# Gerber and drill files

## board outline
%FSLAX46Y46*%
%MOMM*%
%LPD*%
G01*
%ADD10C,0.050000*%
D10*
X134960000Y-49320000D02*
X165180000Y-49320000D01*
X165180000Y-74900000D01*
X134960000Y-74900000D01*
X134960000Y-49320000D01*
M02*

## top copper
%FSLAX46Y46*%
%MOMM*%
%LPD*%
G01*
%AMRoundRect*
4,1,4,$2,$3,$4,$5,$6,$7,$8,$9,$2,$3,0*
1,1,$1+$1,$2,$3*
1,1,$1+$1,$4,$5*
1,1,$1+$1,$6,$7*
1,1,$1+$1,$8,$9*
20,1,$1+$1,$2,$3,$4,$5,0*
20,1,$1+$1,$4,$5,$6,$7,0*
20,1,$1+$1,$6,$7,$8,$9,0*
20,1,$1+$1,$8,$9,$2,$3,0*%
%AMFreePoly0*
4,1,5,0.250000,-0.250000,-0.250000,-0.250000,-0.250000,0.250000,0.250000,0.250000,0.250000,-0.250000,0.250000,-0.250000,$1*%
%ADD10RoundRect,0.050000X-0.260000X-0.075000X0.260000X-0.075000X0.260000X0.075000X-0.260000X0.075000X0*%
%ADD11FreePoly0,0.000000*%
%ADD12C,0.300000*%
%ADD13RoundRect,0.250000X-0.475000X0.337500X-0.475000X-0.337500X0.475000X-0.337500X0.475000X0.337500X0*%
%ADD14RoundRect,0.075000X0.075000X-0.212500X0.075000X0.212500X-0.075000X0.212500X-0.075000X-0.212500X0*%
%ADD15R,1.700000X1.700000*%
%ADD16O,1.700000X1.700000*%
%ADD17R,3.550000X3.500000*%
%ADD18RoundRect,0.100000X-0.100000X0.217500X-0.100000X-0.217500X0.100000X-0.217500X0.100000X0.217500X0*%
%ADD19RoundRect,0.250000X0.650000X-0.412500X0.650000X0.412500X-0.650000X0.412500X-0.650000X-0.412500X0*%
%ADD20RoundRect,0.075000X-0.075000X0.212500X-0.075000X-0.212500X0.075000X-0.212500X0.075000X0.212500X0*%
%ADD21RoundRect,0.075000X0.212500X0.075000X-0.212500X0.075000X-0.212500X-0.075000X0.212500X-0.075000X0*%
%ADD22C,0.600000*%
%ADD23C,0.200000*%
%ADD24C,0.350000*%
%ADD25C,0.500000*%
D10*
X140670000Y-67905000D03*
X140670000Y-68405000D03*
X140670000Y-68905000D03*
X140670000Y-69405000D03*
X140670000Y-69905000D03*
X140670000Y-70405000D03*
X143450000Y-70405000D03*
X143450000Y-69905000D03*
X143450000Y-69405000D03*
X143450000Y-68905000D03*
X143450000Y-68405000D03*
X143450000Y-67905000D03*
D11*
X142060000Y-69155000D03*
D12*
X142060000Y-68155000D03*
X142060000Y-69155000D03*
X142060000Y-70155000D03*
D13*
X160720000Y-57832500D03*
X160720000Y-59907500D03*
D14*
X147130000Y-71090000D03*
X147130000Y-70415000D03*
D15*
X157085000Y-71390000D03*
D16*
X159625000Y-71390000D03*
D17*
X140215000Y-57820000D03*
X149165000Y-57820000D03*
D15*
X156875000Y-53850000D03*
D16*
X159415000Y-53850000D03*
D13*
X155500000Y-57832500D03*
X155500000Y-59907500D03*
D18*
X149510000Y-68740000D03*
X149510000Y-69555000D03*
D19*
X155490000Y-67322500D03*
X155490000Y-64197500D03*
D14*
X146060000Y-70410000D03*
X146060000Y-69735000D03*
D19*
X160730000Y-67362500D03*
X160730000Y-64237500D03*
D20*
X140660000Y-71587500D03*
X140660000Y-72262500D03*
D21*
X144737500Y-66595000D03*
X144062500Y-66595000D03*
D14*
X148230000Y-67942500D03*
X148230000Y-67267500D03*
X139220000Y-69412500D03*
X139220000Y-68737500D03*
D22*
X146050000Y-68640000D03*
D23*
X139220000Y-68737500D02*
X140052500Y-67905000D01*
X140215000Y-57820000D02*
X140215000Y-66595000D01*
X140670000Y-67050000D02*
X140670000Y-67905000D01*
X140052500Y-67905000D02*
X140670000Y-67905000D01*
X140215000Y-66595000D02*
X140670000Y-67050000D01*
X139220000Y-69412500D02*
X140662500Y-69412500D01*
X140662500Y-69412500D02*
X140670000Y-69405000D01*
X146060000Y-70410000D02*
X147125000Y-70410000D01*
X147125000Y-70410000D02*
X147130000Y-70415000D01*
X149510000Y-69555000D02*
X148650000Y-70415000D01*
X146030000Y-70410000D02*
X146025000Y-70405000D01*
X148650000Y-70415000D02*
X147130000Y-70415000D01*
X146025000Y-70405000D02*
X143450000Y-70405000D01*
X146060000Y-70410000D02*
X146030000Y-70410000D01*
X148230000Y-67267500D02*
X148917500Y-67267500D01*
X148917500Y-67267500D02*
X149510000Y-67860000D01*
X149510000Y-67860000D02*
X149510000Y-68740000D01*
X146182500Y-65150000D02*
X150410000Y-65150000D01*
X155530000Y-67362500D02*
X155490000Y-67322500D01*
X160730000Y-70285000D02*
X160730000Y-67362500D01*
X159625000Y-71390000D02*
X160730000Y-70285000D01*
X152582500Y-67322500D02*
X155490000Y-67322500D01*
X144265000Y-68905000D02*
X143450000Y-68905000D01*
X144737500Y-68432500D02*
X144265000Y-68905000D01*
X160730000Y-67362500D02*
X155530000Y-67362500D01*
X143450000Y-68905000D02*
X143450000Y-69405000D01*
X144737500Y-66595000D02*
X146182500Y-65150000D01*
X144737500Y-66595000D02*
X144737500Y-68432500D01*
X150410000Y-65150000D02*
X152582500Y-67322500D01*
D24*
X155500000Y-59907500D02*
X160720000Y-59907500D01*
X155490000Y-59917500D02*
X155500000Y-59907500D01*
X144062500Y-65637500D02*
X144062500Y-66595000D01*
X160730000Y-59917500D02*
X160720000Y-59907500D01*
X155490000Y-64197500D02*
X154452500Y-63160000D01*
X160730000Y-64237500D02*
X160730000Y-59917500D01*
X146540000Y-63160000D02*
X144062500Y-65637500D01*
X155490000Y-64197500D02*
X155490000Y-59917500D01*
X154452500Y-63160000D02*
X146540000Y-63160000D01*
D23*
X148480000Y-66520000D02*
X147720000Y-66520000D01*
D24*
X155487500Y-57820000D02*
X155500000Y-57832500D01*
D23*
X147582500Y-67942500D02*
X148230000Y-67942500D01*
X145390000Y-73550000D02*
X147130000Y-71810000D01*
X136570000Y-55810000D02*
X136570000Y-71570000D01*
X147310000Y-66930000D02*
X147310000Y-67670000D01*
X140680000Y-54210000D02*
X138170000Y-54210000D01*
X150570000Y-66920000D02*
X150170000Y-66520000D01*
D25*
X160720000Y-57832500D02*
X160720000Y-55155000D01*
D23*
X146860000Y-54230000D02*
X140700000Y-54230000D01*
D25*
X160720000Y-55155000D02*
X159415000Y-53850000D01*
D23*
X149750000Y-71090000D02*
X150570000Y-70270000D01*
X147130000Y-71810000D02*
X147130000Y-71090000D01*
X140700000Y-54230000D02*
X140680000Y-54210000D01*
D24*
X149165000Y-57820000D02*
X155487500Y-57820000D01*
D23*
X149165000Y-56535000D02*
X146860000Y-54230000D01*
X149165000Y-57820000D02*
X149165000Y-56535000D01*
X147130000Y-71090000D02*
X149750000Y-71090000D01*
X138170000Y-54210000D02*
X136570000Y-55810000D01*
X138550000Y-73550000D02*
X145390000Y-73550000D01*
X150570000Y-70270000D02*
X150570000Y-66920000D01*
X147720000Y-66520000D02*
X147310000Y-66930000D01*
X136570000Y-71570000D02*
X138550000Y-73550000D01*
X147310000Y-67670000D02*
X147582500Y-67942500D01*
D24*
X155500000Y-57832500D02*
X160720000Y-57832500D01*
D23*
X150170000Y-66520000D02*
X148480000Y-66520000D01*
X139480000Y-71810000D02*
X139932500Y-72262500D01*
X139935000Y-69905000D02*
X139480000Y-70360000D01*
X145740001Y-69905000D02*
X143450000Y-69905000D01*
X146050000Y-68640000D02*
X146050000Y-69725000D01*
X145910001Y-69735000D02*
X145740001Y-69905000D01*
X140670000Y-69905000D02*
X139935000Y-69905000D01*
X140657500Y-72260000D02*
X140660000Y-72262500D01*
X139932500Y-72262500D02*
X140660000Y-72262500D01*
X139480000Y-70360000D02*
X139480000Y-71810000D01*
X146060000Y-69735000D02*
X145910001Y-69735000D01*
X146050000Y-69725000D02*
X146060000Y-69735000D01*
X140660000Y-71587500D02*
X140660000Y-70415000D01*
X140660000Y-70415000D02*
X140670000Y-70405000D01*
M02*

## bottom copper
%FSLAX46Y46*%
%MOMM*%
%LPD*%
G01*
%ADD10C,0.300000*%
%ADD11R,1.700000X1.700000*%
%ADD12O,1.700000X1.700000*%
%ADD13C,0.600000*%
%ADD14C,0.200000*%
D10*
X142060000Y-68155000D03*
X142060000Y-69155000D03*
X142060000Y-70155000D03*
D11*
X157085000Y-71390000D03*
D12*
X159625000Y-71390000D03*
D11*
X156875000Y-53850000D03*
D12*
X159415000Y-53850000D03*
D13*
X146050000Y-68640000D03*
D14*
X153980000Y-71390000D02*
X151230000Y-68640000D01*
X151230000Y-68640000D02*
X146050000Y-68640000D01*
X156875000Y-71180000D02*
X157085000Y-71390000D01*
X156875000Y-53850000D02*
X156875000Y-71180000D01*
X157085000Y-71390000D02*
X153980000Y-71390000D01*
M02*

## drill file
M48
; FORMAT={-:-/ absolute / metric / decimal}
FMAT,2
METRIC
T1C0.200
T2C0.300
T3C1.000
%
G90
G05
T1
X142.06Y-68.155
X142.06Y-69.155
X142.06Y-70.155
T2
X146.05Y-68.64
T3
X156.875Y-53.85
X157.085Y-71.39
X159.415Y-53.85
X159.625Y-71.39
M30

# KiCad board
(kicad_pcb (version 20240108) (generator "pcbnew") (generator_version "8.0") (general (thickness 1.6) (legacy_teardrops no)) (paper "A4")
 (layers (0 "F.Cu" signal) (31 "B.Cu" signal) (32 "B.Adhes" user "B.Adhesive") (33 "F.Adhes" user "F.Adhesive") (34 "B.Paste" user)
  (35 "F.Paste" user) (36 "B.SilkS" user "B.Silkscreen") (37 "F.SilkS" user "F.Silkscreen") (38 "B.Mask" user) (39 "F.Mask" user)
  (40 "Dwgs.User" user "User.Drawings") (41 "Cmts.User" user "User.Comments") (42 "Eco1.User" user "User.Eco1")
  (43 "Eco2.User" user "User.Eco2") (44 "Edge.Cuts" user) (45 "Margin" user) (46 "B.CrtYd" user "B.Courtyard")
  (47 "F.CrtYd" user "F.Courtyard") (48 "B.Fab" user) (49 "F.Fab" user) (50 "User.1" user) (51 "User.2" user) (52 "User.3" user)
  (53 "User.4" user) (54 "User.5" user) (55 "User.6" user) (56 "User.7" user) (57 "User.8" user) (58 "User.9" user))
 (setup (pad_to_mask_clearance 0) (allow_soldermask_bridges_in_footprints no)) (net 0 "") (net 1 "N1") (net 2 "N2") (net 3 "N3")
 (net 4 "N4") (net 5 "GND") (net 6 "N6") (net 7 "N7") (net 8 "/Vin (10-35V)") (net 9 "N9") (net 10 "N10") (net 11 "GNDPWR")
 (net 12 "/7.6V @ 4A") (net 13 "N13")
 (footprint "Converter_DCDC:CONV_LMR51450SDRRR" (layer "F.Cu") (at 142.06 69.155)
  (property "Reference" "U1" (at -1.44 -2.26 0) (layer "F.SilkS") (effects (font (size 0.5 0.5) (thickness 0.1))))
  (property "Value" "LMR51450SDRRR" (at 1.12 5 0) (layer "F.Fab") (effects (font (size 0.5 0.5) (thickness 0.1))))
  (pad "1" smd roundrect (at -1.39 -1.25) (size 0.62 0.25) (layers "F.Cu" "F.Paste") (roundrect_rratio 0.2) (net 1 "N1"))
  (pad "2" smd roundrect (at -1.39 -0.75) (size 0.62 0.25) (layers "F.Cu" "F.Paste") (roundrect_rratio 0.2) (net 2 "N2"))
  (pad "3" smd roundrect (at -1.39 -0.25) (size 0.62 0.25) (layers "F.Cu" "F.Paste") (roundrect_rratio 0.2) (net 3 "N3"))
  (pad "4" smd roundrect (at -1.39 0.25) (size 0.62 0.25) (layers "F.Cu" "F.Paste") (roundrect_rratio 0.2) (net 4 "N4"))
  (pad "5" smd roundrect (at -1.39 0.75) (size 0.62 0.25) (layers "F.Cu" "F.Paste") (roundrect_rratio 0.2) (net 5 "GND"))
  (pad "6" smd roundrect (at -1.39 1.25) (size 0.62 0.25) (layers "F.Cu" "F.Paste") (roundrect_rratio 0.2) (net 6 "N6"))
  (pad "7" smd roundrect (at 1.39 1.25) (size 0.62 0.25) (layers "F.Cu" "F.Paste") (roundrect_rratio 0.2) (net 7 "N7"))
  (pad "8" smd roundrect (at 1.39 0.75) (size 0.62 0.25) (layers "F.Cu" "F.Paste") (roundrect_rratio 0.2) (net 5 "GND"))
  (pad "9" smd roundrect (at 1.39 0.25) (size 0.62 0.25) (layers "F.Cu" "F.Paste") (roundrect_rratio 0.2) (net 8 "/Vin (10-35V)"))
  (pad "10" smd roundrect (at 1.39 -0.25) (size 0.62 0.25) (layers "F.Cu" "F.Paste") (roundrect_rratio 0.2) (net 8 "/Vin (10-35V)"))
  (pad "11" smd roundrect (at 1.39 -0.75) (size 0.62 0.25) (layers "F.Cu" "F.Paste") (roundrect_rratio 0.2) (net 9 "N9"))
  (pad "12" smd roundrect (at 1.39 -1.25) (size 0.62 0.25) (layers "F.Cu" "F.Paste") (roundrect_rratio 0.2) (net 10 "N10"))
  (pad "13" smd custom (at 0 0) (size 0.5 0.5) (layers "F.Cu") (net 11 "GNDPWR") (options (clearance outline) (anchor rect)) (primitives))
  (pad "14" thru_hole circle (at 0 -1) (size 0.3 0.3) (drill 0.2) (layers "*.Cu") (remove_unused_layers no))
  (pad "15" thru_hole circle (at 0 0) (size 0.3 0.3) (drill 0.2) (layers "*.Cu") (remove_unused_layers no))
  (pad "16" thru_hole circle (at 0 1) (size 0.3 0.3) (drill 0.2) (layers "*.Cu") (remove_unused_layers no)))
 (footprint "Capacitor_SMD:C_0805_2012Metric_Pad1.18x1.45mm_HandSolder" (layer "F.Cu") (at 160.72 58.87 -90)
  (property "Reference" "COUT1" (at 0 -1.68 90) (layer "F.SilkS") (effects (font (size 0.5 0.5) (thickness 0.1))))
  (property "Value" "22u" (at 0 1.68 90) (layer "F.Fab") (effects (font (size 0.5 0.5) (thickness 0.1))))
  (pad "1" smd roundrect (at -1.0375 0 270) (size 1.175 1.45) (layers "F.Cu" "F.Paste" "F.Mask") (roundrect_rratio 0.212766)
   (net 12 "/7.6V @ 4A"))
  (pad "2" smd roundrect (at 1.0375 0 270) (size 1.175 1.45) (layers "F.Cu" "F.Paste" "F.Mask") (roundrect_rratio 0.212766)
   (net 11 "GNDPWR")))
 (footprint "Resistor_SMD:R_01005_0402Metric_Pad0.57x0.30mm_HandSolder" (layer "F.Cu") (at 147.13 70.7525 90)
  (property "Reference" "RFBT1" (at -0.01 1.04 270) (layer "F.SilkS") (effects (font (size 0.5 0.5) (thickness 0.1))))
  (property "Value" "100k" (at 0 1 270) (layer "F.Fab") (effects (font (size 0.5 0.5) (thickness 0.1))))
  (pad "" smd roundrect (at -0.3625 0 90) (size 0.41 0.27) (layers "F.Paste") (roundrect_rratio 0.25))
  (pad "" smd roundrect (at 0.3625 0 90) (size 0.41 0.27) (layers "F.Paste") (roundrect_rratio 0.25))
  (pad "1" smd roundrect (at -0.3375 0 90) (size 0.575 0.3) (layers "F.Cu" "F.Mask") (roundrect_rratio 0.25) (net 12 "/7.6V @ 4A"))
  (pad "2" smd roundrect (at 0.3375 0 90) (size 0.575 0.3) (layers "F.Cu" "F.Mask") (roundrect_rratio 0.25) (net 7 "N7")))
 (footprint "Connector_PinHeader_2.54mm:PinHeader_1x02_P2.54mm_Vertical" (layer "F.Cu") (at 157.085 71.39 90)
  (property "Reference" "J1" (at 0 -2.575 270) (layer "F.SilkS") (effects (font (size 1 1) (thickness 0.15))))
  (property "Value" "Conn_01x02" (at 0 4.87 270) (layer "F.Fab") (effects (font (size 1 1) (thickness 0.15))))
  (pad "1" thru_hole rect (at 0 0 90) (size 1.7 1.7) (drill 1) (layers "*.Cu" "*.Mask") (remove_unused_layers no) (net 5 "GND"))
  (pad "2" thru_hole oval (at 0 2.54 90) (size 1.7 1.7) (drill 1) (layers "*.Cu" "*.Mask") (remove_unused_layers no) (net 8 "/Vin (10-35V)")))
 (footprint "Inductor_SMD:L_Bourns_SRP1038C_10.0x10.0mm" (layer "F.Cu") (at 144.69 57.82)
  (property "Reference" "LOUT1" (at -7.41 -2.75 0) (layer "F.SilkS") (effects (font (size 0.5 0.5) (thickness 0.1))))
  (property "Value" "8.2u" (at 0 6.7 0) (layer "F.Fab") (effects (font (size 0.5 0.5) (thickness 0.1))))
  (pad "1" smd rect (at -4.475 0) (size 3.55 3.5) (layers "F.Cu" "F.Paste" "F.Mask") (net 1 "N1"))
  (pad "2" smd rect (at 4.475 0) (size 3.55 3.5) (layers "F.Cu" "F.Paste" "F.Mask") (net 12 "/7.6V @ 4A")))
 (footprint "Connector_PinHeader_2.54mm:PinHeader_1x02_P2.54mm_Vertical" (layer "F.Cu") (at 156.875 53.85 90)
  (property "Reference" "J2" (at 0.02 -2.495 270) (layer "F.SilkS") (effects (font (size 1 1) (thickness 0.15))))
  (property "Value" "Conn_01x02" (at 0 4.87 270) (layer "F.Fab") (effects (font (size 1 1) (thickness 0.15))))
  (pad "1" thru_hole rect (at 0 0 90) (size 1.7 1.7) (drill 1) (layers "*.Cu" "*.Mask") (remove_unused_layers no) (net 5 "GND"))
  (pad "2" thru_hole oval (at 0 2.54 90) (size 1.7 1.7) (drill 1) (layers "*.Cu" "*.Mask") (remove_unused_layers no) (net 12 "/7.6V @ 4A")))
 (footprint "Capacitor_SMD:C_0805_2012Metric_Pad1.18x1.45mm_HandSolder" (layer "F.Cu") (at 155.5 58.87 -90)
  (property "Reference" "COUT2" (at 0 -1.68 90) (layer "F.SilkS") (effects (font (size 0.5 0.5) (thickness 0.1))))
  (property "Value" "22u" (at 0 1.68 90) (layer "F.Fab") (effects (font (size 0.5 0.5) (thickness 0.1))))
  (pad "1" smd roundrect (at -1.0375 0 270) (size 1.175 1.45) (layers "F.Cu" "F.Paste" "F.Mask") (roundrect_rratio 0.212766)
   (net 12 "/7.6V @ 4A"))
  (pad "2" smd roundrect (at 1.0375 0 270) (size 1.175 1.45) (layers "F.Cu" "F.Paste" "F.Mask") (roundrect_rratio 0.212766)
   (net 11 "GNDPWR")))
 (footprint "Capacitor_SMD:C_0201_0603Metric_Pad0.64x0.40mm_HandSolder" (layer "F.Cu") (at 149.51 69.1475 -90)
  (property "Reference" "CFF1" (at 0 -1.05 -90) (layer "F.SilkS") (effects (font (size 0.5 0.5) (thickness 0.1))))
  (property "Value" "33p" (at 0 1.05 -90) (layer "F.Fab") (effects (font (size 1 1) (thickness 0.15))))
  (pad "" smd roundrect (at -0.4325 0 270) (size 0.458 0.36) (layers "F.Paste") (roundrect_rratio 0.25))
  (pad "" smd roundrect (at 0.4325 0 270) (size 0.458 0.36) (layers "F.Paste") (roundrect_rratio 0.25))
  (pad "1" smd roundrect (at -0.4075 0 270) (size 0.635 0.4) (layers "F.Cu" "F.Mask") (roundrect_rratio 0.25) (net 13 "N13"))
  (pad "2" smd roundrect (at 0.4075 0 270) (size 0.635 0.4) (layers "F.Cu" "F.Mask") (roundrect_rratio 0.25) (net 7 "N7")))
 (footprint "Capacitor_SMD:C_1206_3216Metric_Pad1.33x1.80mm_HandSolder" (layer "F.Cu") (at 155.49 65.76 90)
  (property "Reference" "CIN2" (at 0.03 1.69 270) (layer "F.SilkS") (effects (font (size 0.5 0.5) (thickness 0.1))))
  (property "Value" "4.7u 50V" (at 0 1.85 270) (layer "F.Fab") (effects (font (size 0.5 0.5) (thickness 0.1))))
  (pad "1" smd roundrect (at -1.5625 0 90) (size 1.325 1.8) (layers "F.Cu" "F.Paste" "F.Mask") (roundrect_rratio 0.188679)
   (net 8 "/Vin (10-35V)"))
  (pad "2" smd roundrect (at 1.5625 0 90) (size 1.325 1.8) (layers "F.Cu" "F.Paste" "F.Mask") (roundrect_rratio 0.188679) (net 11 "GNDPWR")))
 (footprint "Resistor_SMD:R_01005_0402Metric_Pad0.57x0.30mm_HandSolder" (layer "F.Cu") (at 146.06 70.0725 90)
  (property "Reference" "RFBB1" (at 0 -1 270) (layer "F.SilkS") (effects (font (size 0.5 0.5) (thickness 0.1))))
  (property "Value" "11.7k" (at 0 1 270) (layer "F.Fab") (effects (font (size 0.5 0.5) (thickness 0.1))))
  (pad "" smd roundrect (at -0.3625 0 90) (size 0.41 0.27) (layers "F.Paste") (roundrect_rratio 0.25))
  (pad "" smd roundrect (at 0.3625 0 90) (size 0.41 0.27) (layers "F.Paste") (roundrect_rratio 0.25))
  (pad "1" smd roundrect (at -0.3375 0 90) (size 0.575 0.3) (layers "F.Cu" "F.Mask") (roundrect_rratio 0.25) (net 7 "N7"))
  (pad "2" smd roundrect (at 0.3375 0 90) (size 0.575 0.3) (layers "F.Cu" "F.Mask") (roundrect_rratio 0.25) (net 5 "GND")))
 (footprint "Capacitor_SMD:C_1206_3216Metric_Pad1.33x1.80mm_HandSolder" (layer "F.Cu") (at 160.73 65.8 90)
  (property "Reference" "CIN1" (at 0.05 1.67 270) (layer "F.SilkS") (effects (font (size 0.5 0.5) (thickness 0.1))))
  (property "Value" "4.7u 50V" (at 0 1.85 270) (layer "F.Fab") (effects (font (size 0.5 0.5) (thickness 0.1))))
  (pad "1" smd roundrect (at -1.5625 0 90) (size 1.325 1.8) (layers "F.Cu" "F.Paste" "F.Mask") (roundrect_rratio 0.188679)
   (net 8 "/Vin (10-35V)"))
  (pad "2" smd roundrect (at 1.5625 0 90) (size 1.325 1.8) (layers "F.Cu" "F.Paste" "F.Mask") (roundrect_rratio 0.188679) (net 11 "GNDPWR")))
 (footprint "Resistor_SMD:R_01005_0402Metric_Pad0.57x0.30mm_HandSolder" (layer "F.Cu") (at 140.66 71.925 -90)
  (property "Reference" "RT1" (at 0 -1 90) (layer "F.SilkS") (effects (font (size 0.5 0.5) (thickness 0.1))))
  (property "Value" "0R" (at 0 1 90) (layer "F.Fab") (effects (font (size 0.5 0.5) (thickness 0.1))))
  (pad "" smd roundrect (at -0.3625 0 270) (size 0.41 0.27) (layers "F.Paste") (roundrect_rratio 0.25))
  (pad "" smd roundrect (at 0.3625 0 270) (size 0.41 0.27) (layers "F.Paste") (roundrect_rratio 0.25))
  (pad "1" smd roundrect (at -0.3375 0 270) (size 0.575 0.3) (layers "F.Cu" "F.Mask") (roundrect_rratio 0.25) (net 6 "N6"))
  (pad "2" smd roundrect (at 0.3375 0 270) (size 0.575 0.3) (layers "F.Cu" "F.Mask") (roundrect_rratio 0.25) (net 5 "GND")))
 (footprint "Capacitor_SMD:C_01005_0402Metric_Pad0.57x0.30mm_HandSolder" (layer "F.Cu") (at 144.4 66.595 180)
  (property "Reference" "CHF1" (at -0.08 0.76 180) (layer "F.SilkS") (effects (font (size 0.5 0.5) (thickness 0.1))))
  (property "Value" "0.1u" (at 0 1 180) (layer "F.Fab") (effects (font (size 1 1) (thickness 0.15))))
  (pad "" smd roundrect (at -0.3625 0 180) (size 0.41 0.27) (layers "F.Paste") (roundrect_rratio 0.25))
  (pad "" smd roundrect (at 0.3625 0 180) (size 0.41 0.27) (layers "F.Paste") (roundrect_rratio 0.25))
  (pad "1" smd roundrect (at -0.3375 0 180) (size 0.575 0.3) (layers "F.Cu" "F.Mask") (roundrect_rratio 0.25) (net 8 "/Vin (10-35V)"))
  (pad "2" smd roundrect (at 0.3375 0 180) (size 0.575 0.3) (layers "F.Cu" "F.Mask") (roundrect_rratio 0.25) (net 11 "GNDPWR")))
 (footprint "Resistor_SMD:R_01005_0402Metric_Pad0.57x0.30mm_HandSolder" (layer "F.Cu") (at 148.23 67.605 90)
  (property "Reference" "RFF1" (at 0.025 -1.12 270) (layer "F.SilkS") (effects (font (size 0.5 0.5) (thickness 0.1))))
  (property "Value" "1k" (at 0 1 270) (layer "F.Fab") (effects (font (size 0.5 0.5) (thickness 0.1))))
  (pad "" smd roundrect (at -0.3625 0 90) (size 0.41 0.27) (layers "F.Paste") (roundrect_rratio 0.25))
  (pad "" smd roundrect (at 0.3625 0 90) (size 0.41 0.27) (layers "F.Paste") (roundrect_rratio 0.25))
  (pad "1" smd roundrect (at -0.3375 0 90) (size 0.575 0.3) (layers "F.Cu" "F.Mask") (roundrect_rratio 0.25) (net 12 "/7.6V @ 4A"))
  (pad "2" smd roundrect (at 0.3375 0 90) (size 0.575 0.3) (layers "F.Cu" "F.Mask") (roundrect_rratio 0.25) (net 13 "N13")))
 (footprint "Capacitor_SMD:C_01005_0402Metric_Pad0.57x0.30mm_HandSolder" (layer "F.Cu") (at 139.22 69.075 90)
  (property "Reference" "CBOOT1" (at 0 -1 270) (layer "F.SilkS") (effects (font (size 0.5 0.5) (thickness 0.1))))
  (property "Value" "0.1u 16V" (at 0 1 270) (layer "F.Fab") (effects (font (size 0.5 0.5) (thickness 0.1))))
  (pad "" smd roundrect (at -0.3625 0 90) (size 0.41 0.27) (layers "F.Paste") (roundrect_rratio 0.25))
  (pad "" smd roundrect (at 0.3625 0 90) (size 0.41 0.27) (layers "F.Paste") (roundrect_rratio 0.25))
  (pad "1" smd roundrect (at -0.3375 0 90) (size 0.575 0.3) (layers "F.Cu" "F.Mask") (roundrect_rratio 0.25) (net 4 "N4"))
  (pad "2" smd roundrect (at 0.3375 0 90) (size 0.575 0.3) (layers "F.Cu" "F.Mask") (roundrect_rratio 0.25) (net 1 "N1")))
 (gr_rect (start 134.96 49.32) (end 165.18 74.9) (stroke (width 0.05) (type default)) (fill none) (layer "Edge.Cuts"))
 (segment (start 139.22 68.7375) (end 140.0525 67.905) (width 0.2) (layer "F.Cu") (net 1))
 (segment (start 140.215 57.82) (end 140.215 66.595) (width 0.2) (layer "F.Cu") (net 1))
 (segment (start 140.67 67.05) (end 140.67 67.905) (width 0.2) (layer "F.Cu") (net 1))
 (segment (start 140.0525 67.905) (end 140.67 67.905) (width 0.2) (layer "F.Cu") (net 1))
 (segment (start 140.215 66.595) (end 140.67 67.05) (width 0.2) (layer "F.Cu") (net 1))
 (segment (start 139.22 69.4125) (end 140.6625 69.4125) (width 0.2) (layer "F.Cu") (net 4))
 (segment (start 140.6625 69.4125) (end 140.67 69.405) (width 0.2) (layer "F.Cu") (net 4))
 (segment (start 146.06 70.41) (end 147.125 70.41) (width 0.2) (layer "F.Cu") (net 7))
 (segment (start 147.125 70.41) (end 147.13 70.415) (width 0.2) (layer "F.Cu") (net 7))
 (segment (start 149.51 69.555) (end 148.65 70.415) (width 0.2) (layer "F.Cu") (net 7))
 (segment (start 146.03 70.41) (end 146.025 70.405) (width 0.2) (layer "F.Cu") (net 7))
 (segment (start 148.65 70.415) (end 147.13 70.415) (width 0.2) (layer "F.Cu") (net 7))
 (segment (start 146.025 70.405) (end 143.45 70.405) (width 0.2) (layer "F.Cu") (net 7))
 (segment (start 146.06 70.41) (end 146.03 70.41) (width 0.2) (layer "F.Cu") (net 7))
 (segment (start 148.23 67.2675) (end 148.9175 67.2675) (width 0.2) (layer "F.Cu") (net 13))
 (segment (start 148.9175 67.2675) (end 149.51 67.86) (width 0.2) (layer "F.Cu") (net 13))
 (segment (start 149.51 67.86) (end 149.51 68.74) (width 0.2) (layer "F.Cu") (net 13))
 (segment (start 146.1825 65.15) (end 150.41 65.15) (width 0.2) (layer "F.Cu") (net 8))
 (segment (start 155.53 67.3625) (end 155.49 67.3225) (width 0.2) (layer "F.Cu") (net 8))
 (segment (start 160.73 70.285) (end 160.73 67.3625) (width 0.2) (layer "F.Cu") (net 8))
 (segment (start 159.625 71.39) (end 160.73 70.285) (width 0.2) (layer "F.Cu") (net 8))
 (segment (start 152.5825 67.3225) (end 155.49 67.3225) (width 0.2) (layer "F.Cu") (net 8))
 (segment (start 144.265 68.905) (end 143.45 68.905) (width 0.2) (layer "F.Cu") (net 8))
 (segment (start 144.7375 68.4325) (end 144.265 68.905) (width 0.2) (layer "F.Cu") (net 8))
 (segment (start 160.73 67.3625) (end 155.53 67.3625) (width 0.2) (layer "F.Cu") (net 8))
 (segment (start 143.45 68.905) (end 143.45 69.405) (width 0.2) (layer "F.Cu") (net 8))
 (segment (start 144.7375 66.595) (end 146.1825 65.15) (width 0.2) (layer "F.Cu") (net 8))
 (segment (start 144.7375 66.595) (end 144.7375 68.4325) (width 0.2) (layer "F.Cu") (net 8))
 (segment (start 150.41 65.15) (end 152.5825 67.3225) (width 0.2) (layer "F.Cu") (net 8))
 (segment (start 155.5 59.9075) (end 160.72 59.9075) (width 0.35) (layer "F.Cu") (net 11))
 (segment (start 155.49 59.9175) (end 155.5 59.9075) (width 0.35) (layer "F.Cu") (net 11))
 (segment (start 144.0625 65.6375) (end 144.0625 66.595) (width 0.35) (layer "F.Cu") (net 11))
 (segment (start 160.73 59.9175) (end 160.72 59.9075) (width 0.35) (layer "F.Cu") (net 11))
 (segment (start 155.49 64.1975) (end 154.4525 63.16) (width 0.35) (layer "F.Cu") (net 11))
 (segment (start 160.73 64.2375) (end 160.73 59.9175) (width 0.35) (layer "F.Cu") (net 11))
 (segment (start 146.54 63.16) (end 144.0625 65.6375) (width 0.35) (layer "F.Cu") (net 11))
 (segment (start 155.49 64.1975) (end 155.49 59.9175) (width 0.35) (layer "F.Cu") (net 11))
 (segment (start 154.4525 63.16) (end 146.54 63.16) (width 0.35) (layer "F.Cu") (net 11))
 (segment (start 148.48 66.52) (end 147.72 66.52) (width 0.2) (layer "F.Cu") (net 12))
 (segment (start 155.4875 57.82) (end 155.5 57.8325) (width 0.35) (layer "F.Cu") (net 12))
 (segment (start 147.5825 67.9425) (end 148.23 67.9425) (width 0.2) (layer "F.Cu") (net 12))
 (segment (start 145.39 73.55) (end 147.13 71.81) (width 0.2) (layer "F.Cu") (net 12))
 (segment (start 136.57 55.81) (end 136.57 71.57) (width 0.2) (layer "F.Cu") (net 12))
 (segment (start 147.31 66.93) (end 147.31 67.67) (width 0.2) (layer "F.Cu") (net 12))
 (segment (start 140.68 54.21) (end 138.17 54.21) (width 0.2) (layer "F.Cu") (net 12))
 (segment (start 150.57 66.92) (end 150.17 66.52) (width 0.2) (layer "F.Cu") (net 12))
 (segment (start 160.72 57.8325) (end 160.72 55.155) (width 0.5) (layer "F.Cu") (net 12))
 (segment (start 146.86 54.23) (end 140.7 54.23) (width 0.2) (layer "F.Cu") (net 12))
 (segment (start 160.72 55.155) (end 159.415 53.85) (width 0.5) (layer "F.Cu") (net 12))
 (segment (start 149.75 71.09) (end 150.57 70.27) (width 0.2) (layer "F.Cu") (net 12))
 (segment (start 147.13 71.81) (end 147.13 71.09) (width 0.2) (layer "F.Cu") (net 12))
 (segment (start 140.7 54.23) (end 140.68 54.21) (width 0.2) (layer "F.Cu") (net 12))
 (segment (start 149.165 57.82) (end 155.4875 57.82) (width 0.35) (layer "F.Cu") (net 12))
 (segment (start 149.165 56.535) (end 146.86 54.23) (width 0.2) (layer "F.Cu") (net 12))
 (segment (start 149.165 57.82) (end 149.165 56.535) (width 0.2) (layer "F.Cu") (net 12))
 (segment (start 147.13 71.09) (end 149.75 71.09) (width 0.2) (layer "F.Cu") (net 12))
 (segment (start 138.17 54.21) (end 136.57 55.81) (width 0.2) (layer "F.Cu") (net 12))
 (segment (start 138.55 73.55) (end 145.39 73.55) (width 0.2) (layer "F.Cu") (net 12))
 (segment (start 150.57 70.27) (end 150.57 66.92) (width 0.2) (layer "F.Cu") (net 12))
 (segment (start 147.72 66.52) (end 147.31 66.93) (width 0.2) (layer "F.Cu") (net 12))
 (segment (start 136.57 71.57) (end 138.55 73.55) (width 0.2) (layer "F.Cu") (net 12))
 (segment (start 147.31 67.67) (end 147.5825 67.9425) (width 0.2) (layer "F.Cu") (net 12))
 (segment (start 155.5 57.8325) (end 160.72 57.8325) (width 0.35) (layer "F.Cu") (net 12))
 (segment (start 150.17 66.52) (end 148.48 66.52) (width 0.2) (layer "F.Cu") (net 12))
 (segment (start 139.48 71.81) (end 139.9325 72.2625) (width 0.2) (layer "F.Cu") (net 5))
 (segment (start 139.935 69.905) (end 139.48 70.36) (width 0.2) (layer "F.Cu") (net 5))
 (segment (start 145.740001 69.905) (end 143.45 69.905) (width 0.2) (layer "F.Cu") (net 5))
 (segment (start 146.05 68.64) (end 146.05 69.725) (width 0.2) (layer "F.Cu") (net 5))
 (segment (start 145.910001 69.735) (end 145.740001 69.905) (width 0.2) (layer "F.Cu") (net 5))
 (segment (start 140.67 69.905) (end 139.935 69.905) (width 0.2) (layer "F.Cu") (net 5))
 (segment (start 140.6575 72.26) (end 140.66 72.2625) (width 0.2) (layer "F.Cu") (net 5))
 (segment (start 139.9325 72.2625) (end 140.66 72.2625) (width 0.2) (layer "F.Cu") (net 5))
 (segment (start 139.48 70.36) (end 139.48 71.81) (width 0.2) (layer "F.Cu") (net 5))
 (segment (start 146.06 69.735) (end 145.910001 69.735) (width 0.2) (layer "F.Cu") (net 5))
 (segment (start 146.05 69.725) (end 146.06 69.735) (width 0.2) (layer "F.Cu") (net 5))
 (via (at 146.05 68.64) (size 0.6) (drill 0.3) (layers "F.Cu" "B.Cu") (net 5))
 (segment (start 153.98 71.39) (end 151.23 68.64) (width 0.2) (layer "B.Cu") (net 5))
 (segment (start 151.23 68.64) (end 146.05 68.64) (width 0.2) (layer "B.Cu") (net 5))
 (segment (start 156.875 71.18) (end 157.085 71.39) (width 0.2) (layer "B.Cu") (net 5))
 (segment (start 156.875 53.85) (end 156.875 71.18) (width 0.2) (layer "B.Cu") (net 5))
 (segment (start 157.085 71.39) (end 153.98 71.39) (width 0.2) (layer "B.Cu") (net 5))
 (segment (start 140.66 71.5875) (end 140.66 70.415) (width 0.2) (layer "F.Cu") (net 6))
 (segment (start 140.66 70.415) (end 140.67 70.405) (width 0.2) (layer "F.Cu") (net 6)))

